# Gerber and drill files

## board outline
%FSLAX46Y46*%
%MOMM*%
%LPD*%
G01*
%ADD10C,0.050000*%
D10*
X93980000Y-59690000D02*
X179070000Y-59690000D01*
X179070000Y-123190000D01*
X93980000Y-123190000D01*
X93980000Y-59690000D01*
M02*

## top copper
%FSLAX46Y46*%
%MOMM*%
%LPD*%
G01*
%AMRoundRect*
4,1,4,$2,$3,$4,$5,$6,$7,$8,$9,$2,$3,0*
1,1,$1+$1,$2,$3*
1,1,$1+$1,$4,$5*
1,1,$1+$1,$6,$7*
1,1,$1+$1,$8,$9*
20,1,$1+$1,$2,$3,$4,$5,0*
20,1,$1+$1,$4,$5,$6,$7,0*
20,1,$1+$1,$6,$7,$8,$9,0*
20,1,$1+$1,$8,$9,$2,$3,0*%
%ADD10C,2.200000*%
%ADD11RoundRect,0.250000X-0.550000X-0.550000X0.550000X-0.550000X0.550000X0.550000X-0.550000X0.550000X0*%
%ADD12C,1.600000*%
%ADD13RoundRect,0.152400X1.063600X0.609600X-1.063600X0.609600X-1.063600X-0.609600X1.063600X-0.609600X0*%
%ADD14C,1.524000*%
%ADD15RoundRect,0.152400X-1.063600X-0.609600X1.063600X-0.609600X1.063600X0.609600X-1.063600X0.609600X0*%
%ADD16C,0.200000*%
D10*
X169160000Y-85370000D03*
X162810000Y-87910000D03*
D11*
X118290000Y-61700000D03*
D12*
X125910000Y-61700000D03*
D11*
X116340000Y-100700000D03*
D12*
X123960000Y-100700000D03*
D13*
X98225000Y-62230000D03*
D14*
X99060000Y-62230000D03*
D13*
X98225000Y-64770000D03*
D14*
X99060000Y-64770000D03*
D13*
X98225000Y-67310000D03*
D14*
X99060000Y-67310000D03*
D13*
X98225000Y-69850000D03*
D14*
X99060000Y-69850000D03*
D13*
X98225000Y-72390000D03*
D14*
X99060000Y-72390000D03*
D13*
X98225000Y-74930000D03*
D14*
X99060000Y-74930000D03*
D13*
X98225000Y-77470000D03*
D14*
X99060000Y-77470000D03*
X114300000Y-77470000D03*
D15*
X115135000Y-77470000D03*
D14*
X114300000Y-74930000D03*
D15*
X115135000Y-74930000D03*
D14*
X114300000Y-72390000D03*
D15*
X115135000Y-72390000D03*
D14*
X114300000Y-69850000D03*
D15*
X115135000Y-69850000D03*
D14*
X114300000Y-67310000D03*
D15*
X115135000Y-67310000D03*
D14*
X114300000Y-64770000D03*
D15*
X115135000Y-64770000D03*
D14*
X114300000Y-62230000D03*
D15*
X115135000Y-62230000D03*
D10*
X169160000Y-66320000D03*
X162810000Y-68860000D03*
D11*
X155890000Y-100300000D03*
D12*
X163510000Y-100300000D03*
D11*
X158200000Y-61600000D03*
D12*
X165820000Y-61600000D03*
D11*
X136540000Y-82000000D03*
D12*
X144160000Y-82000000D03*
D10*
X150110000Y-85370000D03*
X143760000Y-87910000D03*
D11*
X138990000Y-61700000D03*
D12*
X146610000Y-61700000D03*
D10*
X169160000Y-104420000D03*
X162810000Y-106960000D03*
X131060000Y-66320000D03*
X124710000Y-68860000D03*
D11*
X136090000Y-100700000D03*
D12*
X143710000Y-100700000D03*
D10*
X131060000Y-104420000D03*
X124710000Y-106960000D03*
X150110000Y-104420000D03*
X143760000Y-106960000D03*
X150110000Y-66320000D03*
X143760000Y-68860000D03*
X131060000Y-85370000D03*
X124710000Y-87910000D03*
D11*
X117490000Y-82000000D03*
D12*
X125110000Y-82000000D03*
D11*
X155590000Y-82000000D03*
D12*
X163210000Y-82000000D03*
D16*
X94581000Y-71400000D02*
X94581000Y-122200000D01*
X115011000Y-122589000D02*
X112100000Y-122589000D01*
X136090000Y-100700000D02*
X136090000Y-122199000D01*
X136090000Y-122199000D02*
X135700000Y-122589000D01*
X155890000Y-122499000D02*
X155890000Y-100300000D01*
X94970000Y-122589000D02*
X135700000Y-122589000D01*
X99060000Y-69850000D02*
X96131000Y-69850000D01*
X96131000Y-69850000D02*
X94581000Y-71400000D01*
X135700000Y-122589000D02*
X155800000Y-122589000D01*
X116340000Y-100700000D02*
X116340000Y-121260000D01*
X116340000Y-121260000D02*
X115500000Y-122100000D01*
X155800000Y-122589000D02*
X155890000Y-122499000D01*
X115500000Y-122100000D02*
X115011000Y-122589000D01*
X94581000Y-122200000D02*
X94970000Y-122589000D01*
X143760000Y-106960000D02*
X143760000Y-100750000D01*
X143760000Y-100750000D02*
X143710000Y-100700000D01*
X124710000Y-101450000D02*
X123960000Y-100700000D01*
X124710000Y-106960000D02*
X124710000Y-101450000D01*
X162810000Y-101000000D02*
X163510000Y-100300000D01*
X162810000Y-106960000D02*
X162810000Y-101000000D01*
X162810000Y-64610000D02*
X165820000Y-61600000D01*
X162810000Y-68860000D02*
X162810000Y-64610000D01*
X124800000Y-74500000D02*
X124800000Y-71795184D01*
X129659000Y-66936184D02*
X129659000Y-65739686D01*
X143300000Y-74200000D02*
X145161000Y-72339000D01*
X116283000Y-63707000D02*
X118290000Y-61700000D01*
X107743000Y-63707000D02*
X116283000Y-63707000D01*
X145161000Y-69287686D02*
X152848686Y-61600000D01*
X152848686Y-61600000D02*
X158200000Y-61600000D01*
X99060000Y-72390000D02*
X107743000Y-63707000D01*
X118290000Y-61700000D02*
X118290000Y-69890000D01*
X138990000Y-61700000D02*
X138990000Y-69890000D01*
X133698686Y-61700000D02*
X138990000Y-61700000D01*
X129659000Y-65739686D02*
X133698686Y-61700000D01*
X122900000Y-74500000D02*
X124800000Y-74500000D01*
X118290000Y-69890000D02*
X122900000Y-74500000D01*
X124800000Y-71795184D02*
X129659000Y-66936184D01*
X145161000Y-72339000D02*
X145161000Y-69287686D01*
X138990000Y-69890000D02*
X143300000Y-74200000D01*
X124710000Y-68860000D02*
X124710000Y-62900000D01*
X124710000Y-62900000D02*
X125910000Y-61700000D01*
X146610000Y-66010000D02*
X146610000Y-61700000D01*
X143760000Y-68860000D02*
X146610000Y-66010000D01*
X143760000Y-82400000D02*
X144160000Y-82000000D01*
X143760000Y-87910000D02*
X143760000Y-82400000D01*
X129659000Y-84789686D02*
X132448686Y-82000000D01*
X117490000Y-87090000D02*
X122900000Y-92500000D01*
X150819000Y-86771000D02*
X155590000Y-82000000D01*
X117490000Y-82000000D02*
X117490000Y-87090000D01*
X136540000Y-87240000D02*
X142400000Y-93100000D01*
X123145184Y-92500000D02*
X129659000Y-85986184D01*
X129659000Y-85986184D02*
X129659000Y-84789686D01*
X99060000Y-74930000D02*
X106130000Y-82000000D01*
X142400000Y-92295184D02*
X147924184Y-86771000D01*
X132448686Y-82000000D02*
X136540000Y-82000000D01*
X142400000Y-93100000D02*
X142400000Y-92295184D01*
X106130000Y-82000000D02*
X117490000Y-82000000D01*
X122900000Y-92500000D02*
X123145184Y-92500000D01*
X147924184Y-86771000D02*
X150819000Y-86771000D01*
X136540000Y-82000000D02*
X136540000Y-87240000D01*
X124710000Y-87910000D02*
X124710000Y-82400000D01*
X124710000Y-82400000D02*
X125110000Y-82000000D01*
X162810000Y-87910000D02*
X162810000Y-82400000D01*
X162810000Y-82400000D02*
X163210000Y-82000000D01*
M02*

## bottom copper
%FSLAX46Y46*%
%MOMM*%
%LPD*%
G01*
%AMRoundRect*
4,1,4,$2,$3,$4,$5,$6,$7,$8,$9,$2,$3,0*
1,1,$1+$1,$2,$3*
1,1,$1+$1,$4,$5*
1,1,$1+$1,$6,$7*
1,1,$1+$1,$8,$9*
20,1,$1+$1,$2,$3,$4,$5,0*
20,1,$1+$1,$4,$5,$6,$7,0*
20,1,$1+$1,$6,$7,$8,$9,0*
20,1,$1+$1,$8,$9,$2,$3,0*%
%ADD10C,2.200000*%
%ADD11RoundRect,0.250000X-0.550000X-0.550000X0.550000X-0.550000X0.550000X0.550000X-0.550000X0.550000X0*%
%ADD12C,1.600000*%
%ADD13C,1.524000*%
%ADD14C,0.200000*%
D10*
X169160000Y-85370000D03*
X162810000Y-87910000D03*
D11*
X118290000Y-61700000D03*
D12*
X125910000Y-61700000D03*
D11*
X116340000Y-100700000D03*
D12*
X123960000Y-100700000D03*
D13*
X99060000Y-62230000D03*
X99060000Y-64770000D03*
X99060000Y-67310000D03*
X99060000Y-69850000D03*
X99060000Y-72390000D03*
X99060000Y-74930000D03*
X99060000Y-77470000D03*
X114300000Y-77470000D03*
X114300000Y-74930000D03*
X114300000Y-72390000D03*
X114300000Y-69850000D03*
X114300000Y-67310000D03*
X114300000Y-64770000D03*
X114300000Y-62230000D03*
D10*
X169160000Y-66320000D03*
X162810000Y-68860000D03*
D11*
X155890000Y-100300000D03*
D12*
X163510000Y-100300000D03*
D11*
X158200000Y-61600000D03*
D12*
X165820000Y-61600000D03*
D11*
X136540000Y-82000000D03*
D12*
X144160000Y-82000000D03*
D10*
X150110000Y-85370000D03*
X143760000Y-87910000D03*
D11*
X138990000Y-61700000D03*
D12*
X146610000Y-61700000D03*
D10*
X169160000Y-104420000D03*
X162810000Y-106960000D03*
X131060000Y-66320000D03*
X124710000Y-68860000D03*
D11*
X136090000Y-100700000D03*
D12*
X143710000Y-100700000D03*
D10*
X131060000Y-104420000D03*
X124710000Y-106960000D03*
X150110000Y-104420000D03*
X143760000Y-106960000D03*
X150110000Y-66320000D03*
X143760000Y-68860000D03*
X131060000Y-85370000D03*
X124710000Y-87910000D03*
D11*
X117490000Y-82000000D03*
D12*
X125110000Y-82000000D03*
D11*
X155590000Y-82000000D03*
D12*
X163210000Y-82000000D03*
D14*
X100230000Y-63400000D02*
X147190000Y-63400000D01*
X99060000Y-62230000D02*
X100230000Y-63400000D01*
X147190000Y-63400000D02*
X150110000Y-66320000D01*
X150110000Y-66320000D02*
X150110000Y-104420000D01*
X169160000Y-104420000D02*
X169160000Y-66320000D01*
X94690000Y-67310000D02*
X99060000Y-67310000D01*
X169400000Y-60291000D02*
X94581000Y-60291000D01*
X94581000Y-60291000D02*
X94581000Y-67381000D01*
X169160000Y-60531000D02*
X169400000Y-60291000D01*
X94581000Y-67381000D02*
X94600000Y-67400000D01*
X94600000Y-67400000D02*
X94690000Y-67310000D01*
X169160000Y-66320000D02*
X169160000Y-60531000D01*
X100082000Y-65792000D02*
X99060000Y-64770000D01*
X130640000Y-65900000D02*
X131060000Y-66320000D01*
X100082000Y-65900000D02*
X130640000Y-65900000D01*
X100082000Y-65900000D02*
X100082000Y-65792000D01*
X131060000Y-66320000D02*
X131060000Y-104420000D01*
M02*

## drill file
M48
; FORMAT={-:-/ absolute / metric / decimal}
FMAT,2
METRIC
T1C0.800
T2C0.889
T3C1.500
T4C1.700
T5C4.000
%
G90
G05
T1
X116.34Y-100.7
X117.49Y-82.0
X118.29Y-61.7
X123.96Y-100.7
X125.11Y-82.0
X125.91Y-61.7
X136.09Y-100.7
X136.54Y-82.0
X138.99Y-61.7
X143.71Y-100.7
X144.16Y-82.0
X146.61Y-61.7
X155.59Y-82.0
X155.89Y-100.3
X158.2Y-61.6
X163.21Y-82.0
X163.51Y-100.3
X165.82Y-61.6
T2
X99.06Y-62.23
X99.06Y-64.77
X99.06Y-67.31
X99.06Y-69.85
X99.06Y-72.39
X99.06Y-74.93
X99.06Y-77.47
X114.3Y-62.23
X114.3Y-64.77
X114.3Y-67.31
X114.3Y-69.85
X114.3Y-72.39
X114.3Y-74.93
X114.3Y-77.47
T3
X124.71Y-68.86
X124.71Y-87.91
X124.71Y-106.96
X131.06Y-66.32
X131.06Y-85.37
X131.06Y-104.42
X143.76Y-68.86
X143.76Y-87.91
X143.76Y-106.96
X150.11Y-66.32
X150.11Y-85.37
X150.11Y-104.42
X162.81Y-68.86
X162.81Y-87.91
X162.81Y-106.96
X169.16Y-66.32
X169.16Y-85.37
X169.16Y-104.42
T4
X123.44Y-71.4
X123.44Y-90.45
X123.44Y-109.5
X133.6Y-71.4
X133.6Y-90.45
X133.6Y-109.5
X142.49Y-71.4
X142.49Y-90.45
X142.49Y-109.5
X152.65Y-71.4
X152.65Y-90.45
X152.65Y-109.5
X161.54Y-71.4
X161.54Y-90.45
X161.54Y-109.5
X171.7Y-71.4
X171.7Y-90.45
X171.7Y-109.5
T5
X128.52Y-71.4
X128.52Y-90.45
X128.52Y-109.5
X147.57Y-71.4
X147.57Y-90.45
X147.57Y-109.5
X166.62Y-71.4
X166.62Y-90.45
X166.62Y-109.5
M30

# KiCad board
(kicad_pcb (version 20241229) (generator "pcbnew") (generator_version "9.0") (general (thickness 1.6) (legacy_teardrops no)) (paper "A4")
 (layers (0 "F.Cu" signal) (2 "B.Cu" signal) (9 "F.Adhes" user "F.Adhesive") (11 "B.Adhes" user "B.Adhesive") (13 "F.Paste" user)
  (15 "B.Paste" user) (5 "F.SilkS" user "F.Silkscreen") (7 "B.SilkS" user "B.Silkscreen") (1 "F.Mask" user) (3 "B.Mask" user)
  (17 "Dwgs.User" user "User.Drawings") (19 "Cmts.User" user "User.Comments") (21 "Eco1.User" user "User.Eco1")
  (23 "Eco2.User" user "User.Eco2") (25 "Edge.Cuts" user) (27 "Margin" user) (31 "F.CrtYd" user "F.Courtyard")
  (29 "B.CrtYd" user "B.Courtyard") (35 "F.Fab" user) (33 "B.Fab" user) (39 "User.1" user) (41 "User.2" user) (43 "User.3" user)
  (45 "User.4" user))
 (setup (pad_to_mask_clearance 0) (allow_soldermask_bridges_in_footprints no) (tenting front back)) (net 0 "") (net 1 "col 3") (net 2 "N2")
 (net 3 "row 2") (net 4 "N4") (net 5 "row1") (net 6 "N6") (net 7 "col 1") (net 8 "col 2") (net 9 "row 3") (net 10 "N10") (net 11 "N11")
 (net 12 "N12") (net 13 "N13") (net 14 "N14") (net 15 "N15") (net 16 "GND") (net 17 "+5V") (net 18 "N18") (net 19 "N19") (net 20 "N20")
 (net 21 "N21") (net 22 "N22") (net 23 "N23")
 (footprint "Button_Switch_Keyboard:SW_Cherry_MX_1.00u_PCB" (layer "F.Cu") (at 169.16 85.37)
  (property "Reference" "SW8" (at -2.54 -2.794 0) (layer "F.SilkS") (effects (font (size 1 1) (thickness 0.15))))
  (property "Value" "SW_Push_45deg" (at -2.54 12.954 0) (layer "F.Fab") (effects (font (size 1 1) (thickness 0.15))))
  (pad "" np_thru_hole circle (at -7.62 5.08) (size 1.7 1.7) (drill 1.7) (layers "*.Cu" "*.Mask"))
  (pad "" np_thru_hole circle (at -2.54 5.08) (size 4 4) (drill 4) (layers "*.Cu" "*.Mask"))
  (pad "" np_thru_hole circle (at 2.54 5.08) (size 1.7 1.7) (drill 1.7) (layers "*.Cu" "*.Mask"))
  (pad "1" thru_hole circle (at 0 0) (size 2.2 2.2) (drill 1.5) (layers "*.Cu" "*.Mask") (remove_unused_layers no) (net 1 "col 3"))
  (pad "2" thru_hole circle (at -6.35 2.54) (size 2.2 2.2) (drill 1.5) (layers "*.Cu" "*.Mask") (remove_unused_layers no) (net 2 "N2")))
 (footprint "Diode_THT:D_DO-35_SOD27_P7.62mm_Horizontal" (layer "F.Cu") (at 118.29 61.7)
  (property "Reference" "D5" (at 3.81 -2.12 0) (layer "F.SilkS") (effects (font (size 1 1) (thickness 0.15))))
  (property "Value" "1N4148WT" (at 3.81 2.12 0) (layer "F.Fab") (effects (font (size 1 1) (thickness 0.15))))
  (pad "1" thru_hole roundrect (at 0 0) (size 1.6 1.6) (drill 0.8) (layers "*.Cu" "*.Mask") (remove_unused_layers no)
   (roundrect_rratio 0.15625) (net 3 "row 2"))
  (pad "2" thru_hole circle (at 7.62 0) (size 1.6 1.6) (drill 0.8) (layers "*.Cu" "*.Mask") (remove_unused_layers no) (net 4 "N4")))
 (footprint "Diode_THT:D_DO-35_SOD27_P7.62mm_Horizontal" (layer "F.Cu") (at 116.34 100.7)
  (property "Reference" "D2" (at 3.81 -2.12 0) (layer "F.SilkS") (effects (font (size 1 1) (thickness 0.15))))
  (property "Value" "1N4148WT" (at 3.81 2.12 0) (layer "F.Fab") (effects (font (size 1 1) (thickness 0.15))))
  (pad "1" thru_hole roundrect (at 0 0) (size 1.6 1.6) (drill 0.8) (layers "*.Cu" "*.Mask") (remove_unused_layers no)
   (roundrect_rratio 0.15625) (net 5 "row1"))
  (pad "2" thru_hole circle (at 7.62 0) (size 1.6 1.6) (drill 0.8) (layers "*.Cu" "*.Mask") (remove_unused_layers no) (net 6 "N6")))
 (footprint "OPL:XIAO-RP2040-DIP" (layer "F.Cu") (at 106.68 69.85)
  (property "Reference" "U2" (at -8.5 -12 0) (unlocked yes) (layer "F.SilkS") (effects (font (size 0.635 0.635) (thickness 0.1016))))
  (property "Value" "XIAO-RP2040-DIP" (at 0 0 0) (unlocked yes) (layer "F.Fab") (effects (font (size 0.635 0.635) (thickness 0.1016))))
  (pad "1" smd roundrect (at -8.455 -7.62 180) (size 2.432 1.524) (layers "F.Cu" "F.Mask") (roundrect_rratio 0.1) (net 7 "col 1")
   (thermal_bridge_angle 45))
  (pad "1" thru_hole circle (at -7.62 -7.62 180) (size 1.524 1.524) (drill 0.889) (layers "*.Cu" "*.Mask") (remove_unused_layers no)
   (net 7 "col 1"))
  (pad "2" smd roundrect (at -8.455 -5.08 180) (size 2.432 1.524) (layers "F.Cu" "F.Mask") (roundrect_rratio 0.1) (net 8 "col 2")
   (thermal_bridge_angle 45))
  (pad "2" thru_hole circle (at -7.62 -5.08 180) (size 1.524 1.524) (drill 0.889) (layers "*.Cu" "*.Mask") (remove_unused_layers no)
   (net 8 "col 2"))
  (pad "3" smd roundrect (at -8.455 -2.54 180) (size 2.432 1.524) (layers "F.Cu" "F.Mask") (roundrect_rratio 0.1) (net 1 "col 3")
   (thermal_bridge_angle 45))
  (pad "3" thru_hole circle (at -7.62 -2.54 180) (size 1.524 1.524) (drill 0.889) (layers "*.Cu" "*.Mask") (remove_unused_layers no)
   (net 1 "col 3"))
  (pad "4" smd roundrect (at -8.455 0 180) (size 2.432 1.524) (layers "F.Cu" "F.Mask") (roundrect_rratio 0.1) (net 5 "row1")
   (thermal_bridge_angle 45))
  (pad "4" thru_hole circle (at -7.62 0 180) (size 1.524 1.524) (drill 0.889) (layers "*.Cu" "*.Mask") (remove_unused_layers no)
   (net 5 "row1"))
  (pad "5" smd roundrect (at -8.455 2.54 180) (size 2.432 1.524) (layers "F.Cu" "F.Mask") (roundrect_rratio 0.1) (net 3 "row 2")
   (thermal_bridge_angle 45))
  (pad "5" thru_hole circle (at -7.62 2.54 180) (size 1.524 1.524) (drill 0.889) (layers "*.Cu" "*.Mask") (remove_unused_layers no)
   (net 3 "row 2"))
  (pad "6" smd roundrect (at -8.455 5.08 180) (size 2.432 1.524) (layers "F.Cu" "F.Mask") (roundrect_rratio 0.1) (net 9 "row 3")
   (thermal_bridge_angle 45))
  (pad "6" thru_hole circle (at -7.62 5.08 180) (size 1.524 1.524) (drill 0.889) (layers "*.Cu" "*.Mask") (remove_unused_layers no)
   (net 9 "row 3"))
  (pad "7" smd roundrect (at -8.455 7.62 180) (size 2.432 1.524) (layers "F.Cu" "F.Mask") (roundrect_rratio 0.1) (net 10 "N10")
   (thermal_bridge_angle 45))
  (pad "7" thru_hole circle (at -7.62 7.62 180) (size 1.524 1.524) (drill 0.889) (layers "*.Cu" "*.Mask") (remove_unused_layers no)
   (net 10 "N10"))
  (pad "8" thru_hole circle (at 7.62 7.62) (size 1.524 1.524) (drill 0.889) (layers "*.Cu" "*.Mask") (remove_unused_layers no)
   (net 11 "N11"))
  (pad "8" smd roundrect (at 8.455 7.62) (size 2.432 1.524) (layers "F.Cu" "F.Mask") (roundrect_rratio 0.1) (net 11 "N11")
   (thermal_bridge_angle 45))
  (pad "9" thru_hole circle (at 7.62 5.08) (size 1.524 1.524) (drill 0.889) (layers "*.Cu" "*.Mask") (remove_unused_layers no)
   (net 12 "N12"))
  (pad "9" smd roundrect (at 8.455 5.08) (size 2.432 1.524) (layers "F.Cu" "F.Mask") (roundrect_rratio 0.1) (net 12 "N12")
   (thermal_bridge_angle 45))
  (pad "10" thru_hole circle (at 7.62 2.54) (size 1.524 1.524) (drill 0.889) (layers "*.Cu" "*.Mask") (remove_unused_layers no)
   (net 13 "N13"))
  (pad "10" smd roundrect (at 8.455 2.54) (size 2.432 1.524) (layers "F.Cu" "F.Mask") (roundrect_rratio 0.1) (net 13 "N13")
   (thermal_bridge_angle 45))
  (pad "11" thru_hole circle (at 7.62 0) (size 1.524 1.524) (drill 0.889) (layers "*.Cu" "*.Mask") (remove_unused_layers no) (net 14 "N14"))
  (pad "11" smd roundrect (at 8.455 0) (size 2.432 1.524) (layers "F.Cu" "F.Mask") (roundrect_rratio 0.1) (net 14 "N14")
   (thermal_bridge_angle 45))
  (pad "12" thru_hole circle (at 7.62 -2.54) (size 1.524 1.524) (drill 0.889) (layers "*.Cu" "*.Mask") (remove_unused_layers no)
   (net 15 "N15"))
  (pad "12" smd roundrect (at 8.455 -2.54) (size 2.432 1.524) (layers "F.Cu" "F.Mask") (roundrect_rratio 0.1) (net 15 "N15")
   (thermal_bridge_angle 45))
  (pad "13" thru_hole circle (at 7.62 -5.08) (size 1.524 1.524) (drill 0.889) (layers "*.Cu" "*.Mask") (remove_unused_layers no)
   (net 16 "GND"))
  (pad "13" smd roundrect (at 8.455 -5.08) (size 2.432 1.524) (layers "F.Cu" "F.Mask") (roundrect_rratio 0.1) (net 16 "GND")
   (thermal_bridge_angle 45))
  (pad "14" thru_hole circle (at 7.62 -7.62) (size 1.524 1.524) (drill 0.889) (layers "*.Cu" "*.Mask") (remove_unused_layers no)
   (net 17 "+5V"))
  (pad "14" smd roundrect (at 8.455 -7.62) (size 2.432 1.524) (layers "F.Cu" "F.Mask") (roundrect_rratio 0.1) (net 17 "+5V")
   (thermal_bridge_angle 45)))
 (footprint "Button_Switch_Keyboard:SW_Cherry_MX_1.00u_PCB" (layer "F.Cu") (at 169.16 66.32)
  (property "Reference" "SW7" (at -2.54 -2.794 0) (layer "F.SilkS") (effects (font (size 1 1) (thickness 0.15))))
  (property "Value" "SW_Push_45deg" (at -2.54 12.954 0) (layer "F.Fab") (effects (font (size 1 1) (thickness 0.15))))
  (pad "" np_thru_hole circle (at -7.62 5.08) (size 1.7 1.7) (drill 1.7) (layers "*.Cu" "*.Mask"))
  (pad "" np_thru_hole circle (at -2.54 5.08) (size 4 4) (drill 4) (layers "*.Cu" "*.Mask"))
  (pad "" np_thru_hole circle (at 2.54 5.08) (size 1.7 1.7) (drill 1.7) (layers "*.Cu" "*.Mask"))
  (pad "1" thru_hole circle (at 0 0) (size 2.2 2.2) (drill 1.5) (layers "*.Cu" "*.Mask") (remove_unused_layers no) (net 1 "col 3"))
  (pad "2" thru_hole circle (at -6.35 2.54) (size 2.2 2.2) (drill 1.5) (layers "*.Cu" "*.Mask") (remove_unused_layers no) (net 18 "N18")))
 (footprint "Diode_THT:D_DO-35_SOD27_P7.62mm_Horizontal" (layer "F.Cu") (at 155.89 100.3)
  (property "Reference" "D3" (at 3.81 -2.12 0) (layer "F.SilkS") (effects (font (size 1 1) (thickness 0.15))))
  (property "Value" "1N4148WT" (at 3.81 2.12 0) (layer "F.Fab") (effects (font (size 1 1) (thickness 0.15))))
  (pad "1" thru_hole roundrect (at 0 0) (size 1.6 1.6) (drill 0.8) (layers "*.Cu" "*.Mask") (remove_unused_layers no)
   (roundrect_rratio 0.15625) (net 5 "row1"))
  (pad "2" thru_hole circle (at 7.62 0) (size 1.6 1.6) (drill 0.8) (layers "*.Cu" "*.Mask") (remove_unused_layers no) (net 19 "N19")))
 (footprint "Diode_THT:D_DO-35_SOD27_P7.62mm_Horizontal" (layer "F.Cu") (at 158.2 61.6)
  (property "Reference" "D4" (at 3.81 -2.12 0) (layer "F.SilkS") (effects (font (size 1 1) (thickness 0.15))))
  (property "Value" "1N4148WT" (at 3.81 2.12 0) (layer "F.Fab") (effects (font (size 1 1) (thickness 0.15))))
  (pad "1" thru_hole roundrect (at 0 0) (size 1.6 1.6) (drill 0.8) (layers "*.Cu" "*.Mask") (remove_unused_layers no)
   (roundrect_rratio 0.15625) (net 3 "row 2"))
  (pad "2" thru_hole circle (at 7.62 0) (size 1.6 1.6) (drill 0.8) (layers "*.Cu" "*.Mask") (remove_unused_layers no) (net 18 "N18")))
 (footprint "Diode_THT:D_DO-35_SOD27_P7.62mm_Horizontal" (layer "F.Cu") (at 136.54 82)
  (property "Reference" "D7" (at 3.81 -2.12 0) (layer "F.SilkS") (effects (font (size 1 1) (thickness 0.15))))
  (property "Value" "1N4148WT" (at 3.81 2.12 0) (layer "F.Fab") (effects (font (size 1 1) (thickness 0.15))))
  (pad "1" thru_hole roundrect (at 0 0) (size 1.6 1.6) (drill 0.8) (layers "*.Cu" "*.Mask") (remove_unused_layers no)
   (roundrect_rratio 0.15625) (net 9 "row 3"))
  (pad "2" thru_hole circle (at 7.62 0) (size 1.6 1.6) (drill 0.8) (layers "*.Cu" "*.Mask") (remove_unused_layers no) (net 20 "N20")))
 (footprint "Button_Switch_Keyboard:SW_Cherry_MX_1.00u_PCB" (layer "F.Cu") (at 150.11 85.37)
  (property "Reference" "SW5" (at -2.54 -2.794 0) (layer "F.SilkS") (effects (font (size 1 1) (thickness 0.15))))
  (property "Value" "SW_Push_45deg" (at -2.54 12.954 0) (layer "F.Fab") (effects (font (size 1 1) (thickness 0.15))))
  (pad "" np_thru_hole circle (at -7.62 5.08) (size 1.7 1.7) (drill 1.7) (layers "*.Cu" "*.Mask"))
  (pad "" np_thru_hole circle (at -2.54 5.08) (size 4 4) (drill 4) (layers "*.Cu" "*.Mask"))
  (pad "" np_thru_hole circle (at 2.54 5.08) (size 1.7 1.7) (drill 1.7) (layers "*.Cu" "*.Mask"))
  (pad "1" thru_hole circle (at 0 0) (size 2.2 2.2) (drill 1.5) (layers "*.Cu" "*.Mask") (remove_unused_layers no) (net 7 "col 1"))
  (pad "2" thru_hole circle (at -6.35 2.54) (size 2.2 2.2) (drill 1.5) (layers "*.Cu" "*.Mask") (remove_unused_layers no) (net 20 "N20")))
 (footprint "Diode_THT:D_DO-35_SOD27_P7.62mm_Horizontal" (layer "F.Cu") (at 138.99 61.7)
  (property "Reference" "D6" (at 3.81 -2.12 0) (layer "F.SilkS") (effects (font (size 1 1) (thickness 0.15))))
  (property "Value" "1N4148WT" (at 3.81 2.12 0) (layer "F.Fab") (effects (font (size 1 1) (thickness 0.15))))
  (pad "1" thru_hole roundrect (at 0 0) (size 1.6 1.6) (drill 0.8) (layers "*.Cu" "*.Mask") (remove_unused_layers no)
   (roundrect_rratio 0.15625) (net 3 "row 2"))
  (pad "2" thru_hole circle (at 7.62 0) (size 1.6 1.6) (drill 0.8) (layers "*.Cu" "*.Mask") (remove_unused_layers no) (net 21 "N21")))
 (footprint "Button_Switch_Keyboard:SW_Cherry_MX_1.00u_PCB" (layer "F.Cu") (at 169.16 104.42)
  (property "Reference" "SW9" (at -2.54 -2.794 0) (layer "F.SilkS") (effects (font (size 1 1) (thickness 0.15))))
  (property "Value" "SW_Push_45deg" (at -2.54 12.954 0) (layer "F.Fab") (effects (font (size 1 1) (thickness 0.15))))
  (pad "" np_thru_hole circle (at -7.62 5.08) (size 1.7 1.7) (drill 1.7) (layers "*.Cu" "*.Mask"))
  (pad "" np_thru_hole circle (at -2.54 5.08) (size 4 4) (drill 4) (layers "*.Cu" "*.Mask"))
  (pad "" np_thru_hole circle (at 2.54 5.08) (size 1.7 1.7) (drill 1.7) (layers "*.Cu" "*.Mask"))
  (pad "1" thru_hole circle (at 0 0) (size 2.2 2.2) (drill 1.5) (layers "*.Cu" "*.Mask") (remove_unused_layers no) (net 1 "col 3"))
  (pad "2" thru_hole circle (at -6.35 2.54) (size 2.2 2.2) (drill 1.5) (layers "*.Cu" "*.Mask") (remove_unused_layers no) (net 19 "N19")))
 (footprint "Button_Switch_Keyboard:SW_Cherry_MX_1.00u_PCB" (layer "F.Cu") (at 131.06 66.32)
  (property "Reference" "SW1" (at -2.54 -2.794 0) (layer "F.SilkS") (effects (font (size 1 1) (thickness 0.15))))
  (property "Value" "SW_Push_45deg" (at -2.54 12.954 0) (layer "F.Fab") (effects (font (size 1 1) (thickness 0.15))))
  (pad "" np_thru_hole circle (at -7.62 5.08) (size 1.7 1.7) (drill 1.7) (layers "*.Cu" "*.Mask"))
  (pad "" np_thru_hole circle (at -2.54 5.08) (size 4 4) (drill 4) (layers "*.Cu" "*.Mask"))
  (pad "" np_thru_hole circle (at 2.54 5.08) (size 1.7 1.7) (drill 1.7) (layers "*.Cu" "*.Mask"))
  (pad "1" thru_hole circle (at 0 0) (size 2.2 2.2) (drill 1.5) (layers "*.Cu" "*.Mask") (remove_unused_layers no) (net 8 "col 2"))
  (pad "2" thru_hole circle (at -6.35 2.54) (size 2.2 2.2) (drill 1.5) (layers "*.Cu" "*.Mask") (remove_unused_layers no) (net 4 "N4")))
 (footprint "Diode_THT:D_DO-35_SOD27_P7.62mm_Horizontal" (layer "F.Cu") (at 136.09 100.7)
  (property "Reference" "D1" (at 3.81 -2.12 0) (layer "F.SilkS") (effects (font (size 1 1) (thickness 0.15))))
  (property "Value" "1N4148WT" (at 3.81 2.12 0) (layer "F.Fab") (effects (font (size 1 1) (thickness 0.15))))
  (pad "1" thru_hole roundrect (at 0 0) (size 1.6 1.6) (drill 0.8) (layers "*.Cu" "*.Mask") (remove_unused_layers no)
   (roundrect_rratio 0.15625) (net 5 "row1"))
  (pad "2" thru_hole circle (at 7.62 0) (size 1.6 1.6) (drill 0.8) (layers "*.Cu" "*.Mask") (remove_unused_layers no) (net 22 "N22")))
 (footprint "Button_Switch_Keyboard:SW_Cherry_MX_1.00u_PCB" (layer "F.Cu") (at 131.06 104.42)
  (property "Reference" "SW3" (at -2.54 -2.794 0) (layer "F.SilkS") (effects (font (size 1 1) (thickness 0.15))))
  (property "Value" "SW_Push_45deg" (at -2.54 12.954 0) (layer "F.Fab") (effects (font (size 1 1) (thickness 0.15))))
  (pad "" np_thru_hole circle (at -7.62 5.08) (size 1.7 1.7) (drill 1.7) (layers "*.Cu" "*.Mask"))
  (pad "" np_thru_hole circle (at -2.54 5.08) (size 4 4) (drill 4) (layers "*.Cu" "*.Mask"))
  (pad "" np_thru_hole circle (at 2.54 5.08) (size 1.7 1.7) (drill 1.7) (layers "*.Cu" "*.Mask"))
  (pad "1" thru_hole circle (at 0 0) (size 2.2 2.2) (drill 1.5) (layers "*.Cu" "*.Mask") (remove_unused_layers no) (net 8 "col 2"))
  (pad "2" thru_hole circle (at -6.35 2.54) (size 2.2 2.2) (drill 1.5) (layers "*.Cu" "*.Mask") (remove_unused_layers no) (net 6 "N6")))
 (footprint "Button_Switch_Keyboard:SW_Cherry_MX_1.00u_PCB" (layer "F.Cu") (at 150.11 104.42)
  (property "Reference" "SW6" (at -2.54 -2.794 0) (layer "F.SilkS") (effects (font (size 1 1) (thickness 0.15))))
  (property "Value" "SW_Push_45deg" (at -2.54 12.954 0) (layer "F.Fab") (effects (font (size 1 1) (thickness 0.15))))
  (pad "" np_thru_hole circle (at -7.62 5.08) (size 1.7 1.7) (drill 1.7) (layers "*.Cu" "*.Mask"))
  (pad "" np_thru_hole circle (at -2.54 5.08) (size 4 4) (drill 4) (layers "*.Cu" "*.Mask"))
  (pad "" np_thru_hole circle (at 2.54 5.08) (size 1.7 1.7) (drill 1.7) (layers "*.Cu" "*.Mask"))
  (pad "1" thru_hole circle (at 0 0) (size 2.2 2.2) (drill 1.5) (layers "*.Cu" "*.Mask") (remove_unused_layers no) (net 7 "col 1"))
  (pad "2" thru_hole circle (at -6.35 2.54) (size 2.2 2.2) (drill 1.5) (layers "*.Cu" "*.Mask") (remove_unused_layers no) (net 22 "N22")))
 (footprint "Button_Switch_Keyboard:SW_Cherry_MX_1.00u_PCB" (layer "F.Cu") (at 150.11 66.32)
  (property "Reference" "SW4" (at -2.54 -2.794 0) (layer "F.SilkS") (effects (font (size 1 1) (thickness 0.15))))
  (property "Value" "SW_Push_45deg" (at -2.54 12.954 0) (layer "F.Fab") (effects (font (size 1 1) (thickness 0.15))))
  (pad "" np_thru_hole circle (at -7.62 5.08) (size 1.7 1.7) (drill 1.7) (layers "*.Cu" "*.Mask"))
  (pad "" np_thru_hole circle (at -2.54 5.08) (size 4 4) (drill 4) (layers "*.Cu" "*.Mask"))
  (pad "" np_thru_hole circle (at 2.54 5.08) (size 1.7 1.7) (drill 1.7) (layers "*.Cu" "*.Mask"))
  (pad "1" thru_hole circle (at 0 0) (size 2.2 2.2) (drill 1.5) (layers "*.Cu" "*.Mask") (remove_unused_layers no) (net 7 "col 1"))
  (pad "2" thru_hole circle (at -6.35 2.54) (size 2.2 2.2) (drill 1.5) (layers "*.Cu" "*.Mask") (remove_unused_layers no) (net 21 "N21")))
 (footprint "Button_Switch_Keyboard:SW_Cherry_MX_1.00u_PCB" (layer "F.Cu") (at 131.06 85.37)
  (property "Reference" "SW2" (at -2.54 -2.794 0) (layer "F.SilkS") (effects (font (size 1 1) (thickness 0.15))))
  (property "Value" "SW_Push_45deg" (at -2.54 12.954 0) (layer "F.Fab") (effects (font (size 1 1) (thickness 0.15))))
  (pad "" np_thru_hole circle (at -7.62 5.08) (size 1.7 1.7) (drill 1.7) (layers "*.Cu" "*.Mask"))
  (pad "" np_thru_hole circle (at -2.54 5.08) (size 4 4) (drill 4) (layers "*.Cu" "*.Mask"))
  (pad "" np_thru_hole circle (at 2.54 5.08) (size 1.7 1.7) (drill 1.7) (layers "*.Cu" "*.Mask"))
  (pad "1" thru_hole circle (at 0 0) (size 2.2 2.2) (drill 1.5) (layers "*.Cu" "*.Mask") (remove_unused_layers no) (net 8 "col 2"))
  (pad "2" thru_hole circle (at -6.35 2.54) (size 2.2 2.2) (drill 1.5) (layers "*.Cu" "*.Mask") (remove_unused_layers no) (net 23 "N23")))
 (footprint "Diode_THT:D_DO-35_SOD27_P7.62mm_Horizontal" (layer "F.Cu") (at 117.49 82)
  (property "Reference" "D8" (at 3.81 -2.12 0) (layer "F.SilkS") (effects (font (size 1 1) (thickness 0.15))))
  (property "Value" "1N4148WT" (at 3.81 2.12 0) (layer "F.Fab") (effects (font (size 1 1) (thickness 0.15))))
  (pad "1" thru_hole roundrect (at 0 0) (size 1.6 1.6) (drill 0.8) (layers "*.Cu" "*.Mask") (remove_unused_layers no)
   (roundrect_rratio 0.15625) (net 9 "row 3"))
  (pad "2" thru_hole circle (at 7.62 0) (size 1.6 1.6) (drill 0.8) (layers "*.Cu" "*.Mask") (remove_unused_layers no) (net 23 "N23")))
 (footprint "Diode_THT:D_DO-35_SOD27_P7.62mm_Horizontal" (layer "F.Cu") (at 155.59 82)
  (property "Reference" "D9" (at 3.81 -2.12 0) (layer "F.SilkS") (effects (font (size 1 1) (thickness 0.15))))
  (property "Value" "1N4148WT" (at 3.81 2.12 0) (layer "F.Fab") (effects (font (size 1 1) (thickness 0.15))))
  (pad "1" thru_hole roundrect (at 0 0) (size 1.6 1.6) (drill 0.8) (layers "*.Cu" "*.Mask") (remove_unused_layers no)
   (roundrect_rratio 0.15625) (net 9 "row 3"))
  (pad "2" thru_hole circle (at 7.62 0) (size 1.6 1.6) (drill 0.8) (layers "*.Cu" "*.Mask") (remove_unused_layers no) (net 2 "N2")))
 (gr_rect (start 93.98 59.69) (end 179.07 123.19) (stroke (width 0.05) (type default)) (fill no) (layer "Edge.Cuts"))
 (segment (start 94.581 71.4) (end 94.581 122.2) (width 0.2) (layer "F.Cu") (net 5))
 (segment (start 115.011 122.589) (end 112.1 122.589) (width 0.2) (layer "F.Cu") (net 5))
 (segment (start 136.09 100.7) (end 136.09 122.199) (width 0.2) (layer "F.Cu") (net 5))
 (segment (start 136.09 122.199) (end 135.7 122.589) (width 0.2) (layer "F.Cu") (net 5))
 (segment (start 155.89 122.499) (end 155.89 100.3) (width 0.2) (layer "F.Cu") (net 5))
 (segment (start 94.97 122.589) (end 135.7 122.589) (width 0.2) (layer "F.Cu") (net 5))
 (segment (start 99.06 69.85) (end 96.131 69.85) (width 0.2) (layer "F.Cu") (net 5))
 (segment (start 96.131 69.85) (end 94.581 71.4) (width 0.2) (layer "F.Cu") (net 5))
 (segment (start 135.7 122.589) (end 155.8 122.589) (width 0.2) (layer "F.Cu") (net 5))
 (segment (start 116.34 100.7) (end 116.34 121.26) (width 0.2) (layer "F.Cu") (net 5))
 (segment (start 116.34 121.26) (end 115.5 122.1) (width 0.2) (layer "F.Cu") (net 5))
 (segment (start 155.8 122.589) (end 155.89 122.499) (width 0.2) (layer "F.Cu") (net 5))
 (segment (start 115.5 122.1) (end 115.011 122.589) (width 0.2) (layer "F.Cu") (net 5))
 (segment (start 94.581 122.2) (end 94.97 122.589) (width 0.2) (layer "F.Cu") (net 5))
 (segment (start 143.76 106.96) (end 143.76 100.75) (width 0.2) (layer "F.Cu") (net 22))
 (segment (start 143.76 100.75) (end 143.71 100.7) (width 0.2) (layer "F.Cu") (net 22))
 (segment (start 124.71 101.45) (end 123.96 100.7) (width 0.2) (layer "F.Cu") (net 6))
 (segment (start 124.71 106.96) (end 124.71 101.45) (width 0.2) (layer "F.Cu") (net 6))
 (segment (start 162.81 101) (end 163.51 100.3) (width 0.2) (layer "F.Cu") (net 19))
 (segment (start 162.81 106.96) (end 162.81 101) (width 0.2) (layer "F.Cu") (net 19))
 (segment (start 162.81 64.61) (end 165.82 61.6) (width 0.2) (layer "F.Cu") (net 18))
 (segment (start 162.81 68.86) (end 162.81 64.61) (width 0.2) (layer "F.Cu") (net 18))
 (segment (start 124.8 74.5) (end 124.8 71.795184) (width 0.2) (layer "F.Cu") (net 3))
 (segment (start 129.659 66.936184) (end 129.659 65.739686) (width 0.2) (layer "F.Cu") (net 3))
 (segment (start 143.3 74.2) (end 145.161 72.339) (width 0.2) (layer "F.Cu") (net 3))
 (segment (start 116.283 63.707) (end 118.29 61.7) (width 0.2) (layer "F.Cu") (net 3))
 (segment (start 107.743 63.707) (end 116.283 63.707) (width 0.2) (layer "F.Cu") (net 3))
 (segment (start 145.161 69.287686) (end 152.848686 61.6) (width 0.2) (layer "F.Cu") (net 3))
 (segment (start 152.848686 61.6) (end 158.2 61.6) (width 0.2) (layer "F.Cu") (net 3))
 (segment (start 99.06 72.39) (end 107.743 63.707) (width 0.2) (layer "F.Cu") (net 3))
 (segment (start 118.29 61.7) (end 118.29 69.89) (width 0.2) (layer "F.Cu") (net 3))
 (segment (start 138.99 61.7) (end 138.99 69.89) (width 0.2) (layer "F.Cu") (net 3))
 (segment (start 133.698686 61.7) (end 138.99 61.7) (width 0.2) (layer "F.Cu") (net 3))
 (segment (start 129.659 65.739686) (end 133.698686 61.7) (width 0.2) (layer "F.Cu") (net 3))
 (segment (start 122.9 74.5) (end 124.8 74.5) (width 0.2) (layer "F.Cu") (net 3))
 (segment (start 118.29 69.89) (end 122.9 74.5) (width 0.2) (layer "F.Cu") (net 3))
 (segment (start 124.8 71.795184) (end 129.659 66.936184) (width 0.2) (layer "F.Cu") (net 3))
 (segment (start 145.161 72.339) (end 145.161 69.287686) (width 0.2) (layer "F.Cu") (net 3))
 (segment (start 138.99 69.89) (end 143.3 74.2) (width 0.2) (layer "F.Cu") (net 3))
 (segment (start 124.71 68.86) (end 124.71 62.9) (width 0.2) (layer "F.Cu") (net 4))
 (segment (start 124.71 62.9) (end 125.91 61.7) (width 0.2) (layer "F.Cu") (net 4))
 (segment (start 146.61 66.01) (end 146.61 61.7) (width 0.2) (layer "F.Cu") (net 21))
 (segment (start 143.76 68.86) (end 146.61 66.01) (width 0.2) (layer "F.Cu") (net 21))
 (segment (start 143.76 82.4) (end 144.16 82) (width 0.2) (layer "F.Cu") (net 20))
 (segment (start 143.76 87.91) (end 143.76 82.4) (width 0.2) (layer "F.Cu") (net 20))
 (segment (start 129.659 84.789686) (end 132.448686 82) (width 0.2) (layer "F.Cu") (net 9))
 (segment (start 117.49 87.09) (end 122.9 92.5) (width 0.2) (layer "F.Cu") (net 9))
 (segment (start 150.819 86.771) (end 155.59 82) (width 0.2) (layer "F.Cu") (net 9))
 (segment (start 117.49 82) (end 117.49 87.09) (width 0.2) (layer "F.Cu") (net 9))
 (segment (start 136.54 87.24) (end 142.4 93.1) (width 0.2) (layer "F.Cu") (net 9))
 (segment (start 123.145184 92.5) (end 129.659 85.986184) (width 0.2) (layer "F.Cu") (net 9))
 (segment (start 129.659 85.986184) (end 129.659 84.789686) (width 0.2) (layer "F.Cu") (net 9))
 (segment (start 99.06 74.93) (end 106.13 82) (width 0.2) (layer "F.Cu") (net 9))
 (segment (start 142.4 92.295184) (end 147.924184 86.771) (width 0.2) (layer "F.Cu") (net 9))
 (segment (start 132.448686 82) (end 136.54 82) (width 0.2) (layer "F.Cu") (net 9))
 (segment (start 142.4 93.1) (end 142.4 92.295184) (width 0.2) (layer "F.Cu") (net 9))
 (segment (start 106.13 82) (end 117.49 82) (width 0.2) (layer "F.Cu") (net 9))
 (segment (start 122.9 92.5) (end 123.145184 92.5) (width 0.2) (layer "F.Cu") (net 9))
 (segment (start 147.924184 86.771) (end 150.819 86.771) (width 0.2) (layer "F.Cu") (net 9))
 (segment (start 136.54 82) (end 136.54 87.24) (width 0.2) (layer "F.Cu") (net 9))
 (segment (start 124.71 87.91) (end 124.71 82.4) (width 0.2) (layer "F.Cu") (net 23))
 (segment (start 124.71 82.4) (end 125.11 82) (width 0.2) (layer "F.Cu") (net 23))
 (segment (start 162.81 87.91) (end 162.81 82.4) (width 0.2) (layer "F.Cu") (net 2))
 (segment (start 162.81 82.4) (end 163.21 82) (width 0.2) (layer "F.Cu") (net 2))
 (segment (start 100.23 63.4) (end 147.19 63.4) (width 0.2) (layer "B.Cu") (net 7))
 (segment (start 99.06 62.23) (end 100.23 63.4) (width 0.2) (layer "B.Cu") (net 7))
 (segment (start 147.19 63.4) (end 150.11 66.32) (width 0.2) (layer "B.Cu") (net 7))
 (segment (start 150.11 66.32) (end 150.11 104.42) (width 0.2) (layer "B.Cu") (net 7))
 (segment (start 169.16 104.42) (end 169.16 66.32) (width 0.2) (layer "B.Cu") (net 1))
 (segment (start 94.69 67.31) (end 99.06 67.31) (width 0.2) (layer "B.Cu") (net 1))
 (segment (start 169.4 60.291) (end 94.581 60.291) (width 0.2) (layer "B.Cu") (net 1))
 (segment (start 94.581 60.291) (end 94.581 67.381) (width 0.2) (layer "B.Cu") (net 1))
 (segment (start 169.16 60.531) (end 169.4 60.291) (width 0.2) (layer "B.Cu") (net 1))
 (segment (start 94.581 67.381) (end 94.6 67.4) (width 0.2) (layer "B.Cu") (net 1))
 (segment (start 94.6 67.4) (end 94.69 67.31) (width 0.2) (layer "B.Cu") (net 1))
 (segment (start 169.16 66.32) (end 169.16 60.531) (width 0.2) (layer "B.Cu") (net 1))
 (segment (start 100.082 65.792) (end 99.06 64.77) (width 0.2) (layer "B.Cu") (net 8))
 (segment (start 130.64 65.9) (end 131.06 66.32) (width 0.2) (layer "B.Cu") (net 8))
 (segment (start 100.082 65.9) (end 130.64 65.9) (width 0.2) (layer "B.Cu") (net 8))
 (segment (start 100.082 65.9) (end 100.082 65.792) (width 0.2) (layer "B.Cu") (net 8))
 (segment (start 131.06 66.32) (end 131.06 104.42) (width 0.2) (layer "B.Cu") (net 8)))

